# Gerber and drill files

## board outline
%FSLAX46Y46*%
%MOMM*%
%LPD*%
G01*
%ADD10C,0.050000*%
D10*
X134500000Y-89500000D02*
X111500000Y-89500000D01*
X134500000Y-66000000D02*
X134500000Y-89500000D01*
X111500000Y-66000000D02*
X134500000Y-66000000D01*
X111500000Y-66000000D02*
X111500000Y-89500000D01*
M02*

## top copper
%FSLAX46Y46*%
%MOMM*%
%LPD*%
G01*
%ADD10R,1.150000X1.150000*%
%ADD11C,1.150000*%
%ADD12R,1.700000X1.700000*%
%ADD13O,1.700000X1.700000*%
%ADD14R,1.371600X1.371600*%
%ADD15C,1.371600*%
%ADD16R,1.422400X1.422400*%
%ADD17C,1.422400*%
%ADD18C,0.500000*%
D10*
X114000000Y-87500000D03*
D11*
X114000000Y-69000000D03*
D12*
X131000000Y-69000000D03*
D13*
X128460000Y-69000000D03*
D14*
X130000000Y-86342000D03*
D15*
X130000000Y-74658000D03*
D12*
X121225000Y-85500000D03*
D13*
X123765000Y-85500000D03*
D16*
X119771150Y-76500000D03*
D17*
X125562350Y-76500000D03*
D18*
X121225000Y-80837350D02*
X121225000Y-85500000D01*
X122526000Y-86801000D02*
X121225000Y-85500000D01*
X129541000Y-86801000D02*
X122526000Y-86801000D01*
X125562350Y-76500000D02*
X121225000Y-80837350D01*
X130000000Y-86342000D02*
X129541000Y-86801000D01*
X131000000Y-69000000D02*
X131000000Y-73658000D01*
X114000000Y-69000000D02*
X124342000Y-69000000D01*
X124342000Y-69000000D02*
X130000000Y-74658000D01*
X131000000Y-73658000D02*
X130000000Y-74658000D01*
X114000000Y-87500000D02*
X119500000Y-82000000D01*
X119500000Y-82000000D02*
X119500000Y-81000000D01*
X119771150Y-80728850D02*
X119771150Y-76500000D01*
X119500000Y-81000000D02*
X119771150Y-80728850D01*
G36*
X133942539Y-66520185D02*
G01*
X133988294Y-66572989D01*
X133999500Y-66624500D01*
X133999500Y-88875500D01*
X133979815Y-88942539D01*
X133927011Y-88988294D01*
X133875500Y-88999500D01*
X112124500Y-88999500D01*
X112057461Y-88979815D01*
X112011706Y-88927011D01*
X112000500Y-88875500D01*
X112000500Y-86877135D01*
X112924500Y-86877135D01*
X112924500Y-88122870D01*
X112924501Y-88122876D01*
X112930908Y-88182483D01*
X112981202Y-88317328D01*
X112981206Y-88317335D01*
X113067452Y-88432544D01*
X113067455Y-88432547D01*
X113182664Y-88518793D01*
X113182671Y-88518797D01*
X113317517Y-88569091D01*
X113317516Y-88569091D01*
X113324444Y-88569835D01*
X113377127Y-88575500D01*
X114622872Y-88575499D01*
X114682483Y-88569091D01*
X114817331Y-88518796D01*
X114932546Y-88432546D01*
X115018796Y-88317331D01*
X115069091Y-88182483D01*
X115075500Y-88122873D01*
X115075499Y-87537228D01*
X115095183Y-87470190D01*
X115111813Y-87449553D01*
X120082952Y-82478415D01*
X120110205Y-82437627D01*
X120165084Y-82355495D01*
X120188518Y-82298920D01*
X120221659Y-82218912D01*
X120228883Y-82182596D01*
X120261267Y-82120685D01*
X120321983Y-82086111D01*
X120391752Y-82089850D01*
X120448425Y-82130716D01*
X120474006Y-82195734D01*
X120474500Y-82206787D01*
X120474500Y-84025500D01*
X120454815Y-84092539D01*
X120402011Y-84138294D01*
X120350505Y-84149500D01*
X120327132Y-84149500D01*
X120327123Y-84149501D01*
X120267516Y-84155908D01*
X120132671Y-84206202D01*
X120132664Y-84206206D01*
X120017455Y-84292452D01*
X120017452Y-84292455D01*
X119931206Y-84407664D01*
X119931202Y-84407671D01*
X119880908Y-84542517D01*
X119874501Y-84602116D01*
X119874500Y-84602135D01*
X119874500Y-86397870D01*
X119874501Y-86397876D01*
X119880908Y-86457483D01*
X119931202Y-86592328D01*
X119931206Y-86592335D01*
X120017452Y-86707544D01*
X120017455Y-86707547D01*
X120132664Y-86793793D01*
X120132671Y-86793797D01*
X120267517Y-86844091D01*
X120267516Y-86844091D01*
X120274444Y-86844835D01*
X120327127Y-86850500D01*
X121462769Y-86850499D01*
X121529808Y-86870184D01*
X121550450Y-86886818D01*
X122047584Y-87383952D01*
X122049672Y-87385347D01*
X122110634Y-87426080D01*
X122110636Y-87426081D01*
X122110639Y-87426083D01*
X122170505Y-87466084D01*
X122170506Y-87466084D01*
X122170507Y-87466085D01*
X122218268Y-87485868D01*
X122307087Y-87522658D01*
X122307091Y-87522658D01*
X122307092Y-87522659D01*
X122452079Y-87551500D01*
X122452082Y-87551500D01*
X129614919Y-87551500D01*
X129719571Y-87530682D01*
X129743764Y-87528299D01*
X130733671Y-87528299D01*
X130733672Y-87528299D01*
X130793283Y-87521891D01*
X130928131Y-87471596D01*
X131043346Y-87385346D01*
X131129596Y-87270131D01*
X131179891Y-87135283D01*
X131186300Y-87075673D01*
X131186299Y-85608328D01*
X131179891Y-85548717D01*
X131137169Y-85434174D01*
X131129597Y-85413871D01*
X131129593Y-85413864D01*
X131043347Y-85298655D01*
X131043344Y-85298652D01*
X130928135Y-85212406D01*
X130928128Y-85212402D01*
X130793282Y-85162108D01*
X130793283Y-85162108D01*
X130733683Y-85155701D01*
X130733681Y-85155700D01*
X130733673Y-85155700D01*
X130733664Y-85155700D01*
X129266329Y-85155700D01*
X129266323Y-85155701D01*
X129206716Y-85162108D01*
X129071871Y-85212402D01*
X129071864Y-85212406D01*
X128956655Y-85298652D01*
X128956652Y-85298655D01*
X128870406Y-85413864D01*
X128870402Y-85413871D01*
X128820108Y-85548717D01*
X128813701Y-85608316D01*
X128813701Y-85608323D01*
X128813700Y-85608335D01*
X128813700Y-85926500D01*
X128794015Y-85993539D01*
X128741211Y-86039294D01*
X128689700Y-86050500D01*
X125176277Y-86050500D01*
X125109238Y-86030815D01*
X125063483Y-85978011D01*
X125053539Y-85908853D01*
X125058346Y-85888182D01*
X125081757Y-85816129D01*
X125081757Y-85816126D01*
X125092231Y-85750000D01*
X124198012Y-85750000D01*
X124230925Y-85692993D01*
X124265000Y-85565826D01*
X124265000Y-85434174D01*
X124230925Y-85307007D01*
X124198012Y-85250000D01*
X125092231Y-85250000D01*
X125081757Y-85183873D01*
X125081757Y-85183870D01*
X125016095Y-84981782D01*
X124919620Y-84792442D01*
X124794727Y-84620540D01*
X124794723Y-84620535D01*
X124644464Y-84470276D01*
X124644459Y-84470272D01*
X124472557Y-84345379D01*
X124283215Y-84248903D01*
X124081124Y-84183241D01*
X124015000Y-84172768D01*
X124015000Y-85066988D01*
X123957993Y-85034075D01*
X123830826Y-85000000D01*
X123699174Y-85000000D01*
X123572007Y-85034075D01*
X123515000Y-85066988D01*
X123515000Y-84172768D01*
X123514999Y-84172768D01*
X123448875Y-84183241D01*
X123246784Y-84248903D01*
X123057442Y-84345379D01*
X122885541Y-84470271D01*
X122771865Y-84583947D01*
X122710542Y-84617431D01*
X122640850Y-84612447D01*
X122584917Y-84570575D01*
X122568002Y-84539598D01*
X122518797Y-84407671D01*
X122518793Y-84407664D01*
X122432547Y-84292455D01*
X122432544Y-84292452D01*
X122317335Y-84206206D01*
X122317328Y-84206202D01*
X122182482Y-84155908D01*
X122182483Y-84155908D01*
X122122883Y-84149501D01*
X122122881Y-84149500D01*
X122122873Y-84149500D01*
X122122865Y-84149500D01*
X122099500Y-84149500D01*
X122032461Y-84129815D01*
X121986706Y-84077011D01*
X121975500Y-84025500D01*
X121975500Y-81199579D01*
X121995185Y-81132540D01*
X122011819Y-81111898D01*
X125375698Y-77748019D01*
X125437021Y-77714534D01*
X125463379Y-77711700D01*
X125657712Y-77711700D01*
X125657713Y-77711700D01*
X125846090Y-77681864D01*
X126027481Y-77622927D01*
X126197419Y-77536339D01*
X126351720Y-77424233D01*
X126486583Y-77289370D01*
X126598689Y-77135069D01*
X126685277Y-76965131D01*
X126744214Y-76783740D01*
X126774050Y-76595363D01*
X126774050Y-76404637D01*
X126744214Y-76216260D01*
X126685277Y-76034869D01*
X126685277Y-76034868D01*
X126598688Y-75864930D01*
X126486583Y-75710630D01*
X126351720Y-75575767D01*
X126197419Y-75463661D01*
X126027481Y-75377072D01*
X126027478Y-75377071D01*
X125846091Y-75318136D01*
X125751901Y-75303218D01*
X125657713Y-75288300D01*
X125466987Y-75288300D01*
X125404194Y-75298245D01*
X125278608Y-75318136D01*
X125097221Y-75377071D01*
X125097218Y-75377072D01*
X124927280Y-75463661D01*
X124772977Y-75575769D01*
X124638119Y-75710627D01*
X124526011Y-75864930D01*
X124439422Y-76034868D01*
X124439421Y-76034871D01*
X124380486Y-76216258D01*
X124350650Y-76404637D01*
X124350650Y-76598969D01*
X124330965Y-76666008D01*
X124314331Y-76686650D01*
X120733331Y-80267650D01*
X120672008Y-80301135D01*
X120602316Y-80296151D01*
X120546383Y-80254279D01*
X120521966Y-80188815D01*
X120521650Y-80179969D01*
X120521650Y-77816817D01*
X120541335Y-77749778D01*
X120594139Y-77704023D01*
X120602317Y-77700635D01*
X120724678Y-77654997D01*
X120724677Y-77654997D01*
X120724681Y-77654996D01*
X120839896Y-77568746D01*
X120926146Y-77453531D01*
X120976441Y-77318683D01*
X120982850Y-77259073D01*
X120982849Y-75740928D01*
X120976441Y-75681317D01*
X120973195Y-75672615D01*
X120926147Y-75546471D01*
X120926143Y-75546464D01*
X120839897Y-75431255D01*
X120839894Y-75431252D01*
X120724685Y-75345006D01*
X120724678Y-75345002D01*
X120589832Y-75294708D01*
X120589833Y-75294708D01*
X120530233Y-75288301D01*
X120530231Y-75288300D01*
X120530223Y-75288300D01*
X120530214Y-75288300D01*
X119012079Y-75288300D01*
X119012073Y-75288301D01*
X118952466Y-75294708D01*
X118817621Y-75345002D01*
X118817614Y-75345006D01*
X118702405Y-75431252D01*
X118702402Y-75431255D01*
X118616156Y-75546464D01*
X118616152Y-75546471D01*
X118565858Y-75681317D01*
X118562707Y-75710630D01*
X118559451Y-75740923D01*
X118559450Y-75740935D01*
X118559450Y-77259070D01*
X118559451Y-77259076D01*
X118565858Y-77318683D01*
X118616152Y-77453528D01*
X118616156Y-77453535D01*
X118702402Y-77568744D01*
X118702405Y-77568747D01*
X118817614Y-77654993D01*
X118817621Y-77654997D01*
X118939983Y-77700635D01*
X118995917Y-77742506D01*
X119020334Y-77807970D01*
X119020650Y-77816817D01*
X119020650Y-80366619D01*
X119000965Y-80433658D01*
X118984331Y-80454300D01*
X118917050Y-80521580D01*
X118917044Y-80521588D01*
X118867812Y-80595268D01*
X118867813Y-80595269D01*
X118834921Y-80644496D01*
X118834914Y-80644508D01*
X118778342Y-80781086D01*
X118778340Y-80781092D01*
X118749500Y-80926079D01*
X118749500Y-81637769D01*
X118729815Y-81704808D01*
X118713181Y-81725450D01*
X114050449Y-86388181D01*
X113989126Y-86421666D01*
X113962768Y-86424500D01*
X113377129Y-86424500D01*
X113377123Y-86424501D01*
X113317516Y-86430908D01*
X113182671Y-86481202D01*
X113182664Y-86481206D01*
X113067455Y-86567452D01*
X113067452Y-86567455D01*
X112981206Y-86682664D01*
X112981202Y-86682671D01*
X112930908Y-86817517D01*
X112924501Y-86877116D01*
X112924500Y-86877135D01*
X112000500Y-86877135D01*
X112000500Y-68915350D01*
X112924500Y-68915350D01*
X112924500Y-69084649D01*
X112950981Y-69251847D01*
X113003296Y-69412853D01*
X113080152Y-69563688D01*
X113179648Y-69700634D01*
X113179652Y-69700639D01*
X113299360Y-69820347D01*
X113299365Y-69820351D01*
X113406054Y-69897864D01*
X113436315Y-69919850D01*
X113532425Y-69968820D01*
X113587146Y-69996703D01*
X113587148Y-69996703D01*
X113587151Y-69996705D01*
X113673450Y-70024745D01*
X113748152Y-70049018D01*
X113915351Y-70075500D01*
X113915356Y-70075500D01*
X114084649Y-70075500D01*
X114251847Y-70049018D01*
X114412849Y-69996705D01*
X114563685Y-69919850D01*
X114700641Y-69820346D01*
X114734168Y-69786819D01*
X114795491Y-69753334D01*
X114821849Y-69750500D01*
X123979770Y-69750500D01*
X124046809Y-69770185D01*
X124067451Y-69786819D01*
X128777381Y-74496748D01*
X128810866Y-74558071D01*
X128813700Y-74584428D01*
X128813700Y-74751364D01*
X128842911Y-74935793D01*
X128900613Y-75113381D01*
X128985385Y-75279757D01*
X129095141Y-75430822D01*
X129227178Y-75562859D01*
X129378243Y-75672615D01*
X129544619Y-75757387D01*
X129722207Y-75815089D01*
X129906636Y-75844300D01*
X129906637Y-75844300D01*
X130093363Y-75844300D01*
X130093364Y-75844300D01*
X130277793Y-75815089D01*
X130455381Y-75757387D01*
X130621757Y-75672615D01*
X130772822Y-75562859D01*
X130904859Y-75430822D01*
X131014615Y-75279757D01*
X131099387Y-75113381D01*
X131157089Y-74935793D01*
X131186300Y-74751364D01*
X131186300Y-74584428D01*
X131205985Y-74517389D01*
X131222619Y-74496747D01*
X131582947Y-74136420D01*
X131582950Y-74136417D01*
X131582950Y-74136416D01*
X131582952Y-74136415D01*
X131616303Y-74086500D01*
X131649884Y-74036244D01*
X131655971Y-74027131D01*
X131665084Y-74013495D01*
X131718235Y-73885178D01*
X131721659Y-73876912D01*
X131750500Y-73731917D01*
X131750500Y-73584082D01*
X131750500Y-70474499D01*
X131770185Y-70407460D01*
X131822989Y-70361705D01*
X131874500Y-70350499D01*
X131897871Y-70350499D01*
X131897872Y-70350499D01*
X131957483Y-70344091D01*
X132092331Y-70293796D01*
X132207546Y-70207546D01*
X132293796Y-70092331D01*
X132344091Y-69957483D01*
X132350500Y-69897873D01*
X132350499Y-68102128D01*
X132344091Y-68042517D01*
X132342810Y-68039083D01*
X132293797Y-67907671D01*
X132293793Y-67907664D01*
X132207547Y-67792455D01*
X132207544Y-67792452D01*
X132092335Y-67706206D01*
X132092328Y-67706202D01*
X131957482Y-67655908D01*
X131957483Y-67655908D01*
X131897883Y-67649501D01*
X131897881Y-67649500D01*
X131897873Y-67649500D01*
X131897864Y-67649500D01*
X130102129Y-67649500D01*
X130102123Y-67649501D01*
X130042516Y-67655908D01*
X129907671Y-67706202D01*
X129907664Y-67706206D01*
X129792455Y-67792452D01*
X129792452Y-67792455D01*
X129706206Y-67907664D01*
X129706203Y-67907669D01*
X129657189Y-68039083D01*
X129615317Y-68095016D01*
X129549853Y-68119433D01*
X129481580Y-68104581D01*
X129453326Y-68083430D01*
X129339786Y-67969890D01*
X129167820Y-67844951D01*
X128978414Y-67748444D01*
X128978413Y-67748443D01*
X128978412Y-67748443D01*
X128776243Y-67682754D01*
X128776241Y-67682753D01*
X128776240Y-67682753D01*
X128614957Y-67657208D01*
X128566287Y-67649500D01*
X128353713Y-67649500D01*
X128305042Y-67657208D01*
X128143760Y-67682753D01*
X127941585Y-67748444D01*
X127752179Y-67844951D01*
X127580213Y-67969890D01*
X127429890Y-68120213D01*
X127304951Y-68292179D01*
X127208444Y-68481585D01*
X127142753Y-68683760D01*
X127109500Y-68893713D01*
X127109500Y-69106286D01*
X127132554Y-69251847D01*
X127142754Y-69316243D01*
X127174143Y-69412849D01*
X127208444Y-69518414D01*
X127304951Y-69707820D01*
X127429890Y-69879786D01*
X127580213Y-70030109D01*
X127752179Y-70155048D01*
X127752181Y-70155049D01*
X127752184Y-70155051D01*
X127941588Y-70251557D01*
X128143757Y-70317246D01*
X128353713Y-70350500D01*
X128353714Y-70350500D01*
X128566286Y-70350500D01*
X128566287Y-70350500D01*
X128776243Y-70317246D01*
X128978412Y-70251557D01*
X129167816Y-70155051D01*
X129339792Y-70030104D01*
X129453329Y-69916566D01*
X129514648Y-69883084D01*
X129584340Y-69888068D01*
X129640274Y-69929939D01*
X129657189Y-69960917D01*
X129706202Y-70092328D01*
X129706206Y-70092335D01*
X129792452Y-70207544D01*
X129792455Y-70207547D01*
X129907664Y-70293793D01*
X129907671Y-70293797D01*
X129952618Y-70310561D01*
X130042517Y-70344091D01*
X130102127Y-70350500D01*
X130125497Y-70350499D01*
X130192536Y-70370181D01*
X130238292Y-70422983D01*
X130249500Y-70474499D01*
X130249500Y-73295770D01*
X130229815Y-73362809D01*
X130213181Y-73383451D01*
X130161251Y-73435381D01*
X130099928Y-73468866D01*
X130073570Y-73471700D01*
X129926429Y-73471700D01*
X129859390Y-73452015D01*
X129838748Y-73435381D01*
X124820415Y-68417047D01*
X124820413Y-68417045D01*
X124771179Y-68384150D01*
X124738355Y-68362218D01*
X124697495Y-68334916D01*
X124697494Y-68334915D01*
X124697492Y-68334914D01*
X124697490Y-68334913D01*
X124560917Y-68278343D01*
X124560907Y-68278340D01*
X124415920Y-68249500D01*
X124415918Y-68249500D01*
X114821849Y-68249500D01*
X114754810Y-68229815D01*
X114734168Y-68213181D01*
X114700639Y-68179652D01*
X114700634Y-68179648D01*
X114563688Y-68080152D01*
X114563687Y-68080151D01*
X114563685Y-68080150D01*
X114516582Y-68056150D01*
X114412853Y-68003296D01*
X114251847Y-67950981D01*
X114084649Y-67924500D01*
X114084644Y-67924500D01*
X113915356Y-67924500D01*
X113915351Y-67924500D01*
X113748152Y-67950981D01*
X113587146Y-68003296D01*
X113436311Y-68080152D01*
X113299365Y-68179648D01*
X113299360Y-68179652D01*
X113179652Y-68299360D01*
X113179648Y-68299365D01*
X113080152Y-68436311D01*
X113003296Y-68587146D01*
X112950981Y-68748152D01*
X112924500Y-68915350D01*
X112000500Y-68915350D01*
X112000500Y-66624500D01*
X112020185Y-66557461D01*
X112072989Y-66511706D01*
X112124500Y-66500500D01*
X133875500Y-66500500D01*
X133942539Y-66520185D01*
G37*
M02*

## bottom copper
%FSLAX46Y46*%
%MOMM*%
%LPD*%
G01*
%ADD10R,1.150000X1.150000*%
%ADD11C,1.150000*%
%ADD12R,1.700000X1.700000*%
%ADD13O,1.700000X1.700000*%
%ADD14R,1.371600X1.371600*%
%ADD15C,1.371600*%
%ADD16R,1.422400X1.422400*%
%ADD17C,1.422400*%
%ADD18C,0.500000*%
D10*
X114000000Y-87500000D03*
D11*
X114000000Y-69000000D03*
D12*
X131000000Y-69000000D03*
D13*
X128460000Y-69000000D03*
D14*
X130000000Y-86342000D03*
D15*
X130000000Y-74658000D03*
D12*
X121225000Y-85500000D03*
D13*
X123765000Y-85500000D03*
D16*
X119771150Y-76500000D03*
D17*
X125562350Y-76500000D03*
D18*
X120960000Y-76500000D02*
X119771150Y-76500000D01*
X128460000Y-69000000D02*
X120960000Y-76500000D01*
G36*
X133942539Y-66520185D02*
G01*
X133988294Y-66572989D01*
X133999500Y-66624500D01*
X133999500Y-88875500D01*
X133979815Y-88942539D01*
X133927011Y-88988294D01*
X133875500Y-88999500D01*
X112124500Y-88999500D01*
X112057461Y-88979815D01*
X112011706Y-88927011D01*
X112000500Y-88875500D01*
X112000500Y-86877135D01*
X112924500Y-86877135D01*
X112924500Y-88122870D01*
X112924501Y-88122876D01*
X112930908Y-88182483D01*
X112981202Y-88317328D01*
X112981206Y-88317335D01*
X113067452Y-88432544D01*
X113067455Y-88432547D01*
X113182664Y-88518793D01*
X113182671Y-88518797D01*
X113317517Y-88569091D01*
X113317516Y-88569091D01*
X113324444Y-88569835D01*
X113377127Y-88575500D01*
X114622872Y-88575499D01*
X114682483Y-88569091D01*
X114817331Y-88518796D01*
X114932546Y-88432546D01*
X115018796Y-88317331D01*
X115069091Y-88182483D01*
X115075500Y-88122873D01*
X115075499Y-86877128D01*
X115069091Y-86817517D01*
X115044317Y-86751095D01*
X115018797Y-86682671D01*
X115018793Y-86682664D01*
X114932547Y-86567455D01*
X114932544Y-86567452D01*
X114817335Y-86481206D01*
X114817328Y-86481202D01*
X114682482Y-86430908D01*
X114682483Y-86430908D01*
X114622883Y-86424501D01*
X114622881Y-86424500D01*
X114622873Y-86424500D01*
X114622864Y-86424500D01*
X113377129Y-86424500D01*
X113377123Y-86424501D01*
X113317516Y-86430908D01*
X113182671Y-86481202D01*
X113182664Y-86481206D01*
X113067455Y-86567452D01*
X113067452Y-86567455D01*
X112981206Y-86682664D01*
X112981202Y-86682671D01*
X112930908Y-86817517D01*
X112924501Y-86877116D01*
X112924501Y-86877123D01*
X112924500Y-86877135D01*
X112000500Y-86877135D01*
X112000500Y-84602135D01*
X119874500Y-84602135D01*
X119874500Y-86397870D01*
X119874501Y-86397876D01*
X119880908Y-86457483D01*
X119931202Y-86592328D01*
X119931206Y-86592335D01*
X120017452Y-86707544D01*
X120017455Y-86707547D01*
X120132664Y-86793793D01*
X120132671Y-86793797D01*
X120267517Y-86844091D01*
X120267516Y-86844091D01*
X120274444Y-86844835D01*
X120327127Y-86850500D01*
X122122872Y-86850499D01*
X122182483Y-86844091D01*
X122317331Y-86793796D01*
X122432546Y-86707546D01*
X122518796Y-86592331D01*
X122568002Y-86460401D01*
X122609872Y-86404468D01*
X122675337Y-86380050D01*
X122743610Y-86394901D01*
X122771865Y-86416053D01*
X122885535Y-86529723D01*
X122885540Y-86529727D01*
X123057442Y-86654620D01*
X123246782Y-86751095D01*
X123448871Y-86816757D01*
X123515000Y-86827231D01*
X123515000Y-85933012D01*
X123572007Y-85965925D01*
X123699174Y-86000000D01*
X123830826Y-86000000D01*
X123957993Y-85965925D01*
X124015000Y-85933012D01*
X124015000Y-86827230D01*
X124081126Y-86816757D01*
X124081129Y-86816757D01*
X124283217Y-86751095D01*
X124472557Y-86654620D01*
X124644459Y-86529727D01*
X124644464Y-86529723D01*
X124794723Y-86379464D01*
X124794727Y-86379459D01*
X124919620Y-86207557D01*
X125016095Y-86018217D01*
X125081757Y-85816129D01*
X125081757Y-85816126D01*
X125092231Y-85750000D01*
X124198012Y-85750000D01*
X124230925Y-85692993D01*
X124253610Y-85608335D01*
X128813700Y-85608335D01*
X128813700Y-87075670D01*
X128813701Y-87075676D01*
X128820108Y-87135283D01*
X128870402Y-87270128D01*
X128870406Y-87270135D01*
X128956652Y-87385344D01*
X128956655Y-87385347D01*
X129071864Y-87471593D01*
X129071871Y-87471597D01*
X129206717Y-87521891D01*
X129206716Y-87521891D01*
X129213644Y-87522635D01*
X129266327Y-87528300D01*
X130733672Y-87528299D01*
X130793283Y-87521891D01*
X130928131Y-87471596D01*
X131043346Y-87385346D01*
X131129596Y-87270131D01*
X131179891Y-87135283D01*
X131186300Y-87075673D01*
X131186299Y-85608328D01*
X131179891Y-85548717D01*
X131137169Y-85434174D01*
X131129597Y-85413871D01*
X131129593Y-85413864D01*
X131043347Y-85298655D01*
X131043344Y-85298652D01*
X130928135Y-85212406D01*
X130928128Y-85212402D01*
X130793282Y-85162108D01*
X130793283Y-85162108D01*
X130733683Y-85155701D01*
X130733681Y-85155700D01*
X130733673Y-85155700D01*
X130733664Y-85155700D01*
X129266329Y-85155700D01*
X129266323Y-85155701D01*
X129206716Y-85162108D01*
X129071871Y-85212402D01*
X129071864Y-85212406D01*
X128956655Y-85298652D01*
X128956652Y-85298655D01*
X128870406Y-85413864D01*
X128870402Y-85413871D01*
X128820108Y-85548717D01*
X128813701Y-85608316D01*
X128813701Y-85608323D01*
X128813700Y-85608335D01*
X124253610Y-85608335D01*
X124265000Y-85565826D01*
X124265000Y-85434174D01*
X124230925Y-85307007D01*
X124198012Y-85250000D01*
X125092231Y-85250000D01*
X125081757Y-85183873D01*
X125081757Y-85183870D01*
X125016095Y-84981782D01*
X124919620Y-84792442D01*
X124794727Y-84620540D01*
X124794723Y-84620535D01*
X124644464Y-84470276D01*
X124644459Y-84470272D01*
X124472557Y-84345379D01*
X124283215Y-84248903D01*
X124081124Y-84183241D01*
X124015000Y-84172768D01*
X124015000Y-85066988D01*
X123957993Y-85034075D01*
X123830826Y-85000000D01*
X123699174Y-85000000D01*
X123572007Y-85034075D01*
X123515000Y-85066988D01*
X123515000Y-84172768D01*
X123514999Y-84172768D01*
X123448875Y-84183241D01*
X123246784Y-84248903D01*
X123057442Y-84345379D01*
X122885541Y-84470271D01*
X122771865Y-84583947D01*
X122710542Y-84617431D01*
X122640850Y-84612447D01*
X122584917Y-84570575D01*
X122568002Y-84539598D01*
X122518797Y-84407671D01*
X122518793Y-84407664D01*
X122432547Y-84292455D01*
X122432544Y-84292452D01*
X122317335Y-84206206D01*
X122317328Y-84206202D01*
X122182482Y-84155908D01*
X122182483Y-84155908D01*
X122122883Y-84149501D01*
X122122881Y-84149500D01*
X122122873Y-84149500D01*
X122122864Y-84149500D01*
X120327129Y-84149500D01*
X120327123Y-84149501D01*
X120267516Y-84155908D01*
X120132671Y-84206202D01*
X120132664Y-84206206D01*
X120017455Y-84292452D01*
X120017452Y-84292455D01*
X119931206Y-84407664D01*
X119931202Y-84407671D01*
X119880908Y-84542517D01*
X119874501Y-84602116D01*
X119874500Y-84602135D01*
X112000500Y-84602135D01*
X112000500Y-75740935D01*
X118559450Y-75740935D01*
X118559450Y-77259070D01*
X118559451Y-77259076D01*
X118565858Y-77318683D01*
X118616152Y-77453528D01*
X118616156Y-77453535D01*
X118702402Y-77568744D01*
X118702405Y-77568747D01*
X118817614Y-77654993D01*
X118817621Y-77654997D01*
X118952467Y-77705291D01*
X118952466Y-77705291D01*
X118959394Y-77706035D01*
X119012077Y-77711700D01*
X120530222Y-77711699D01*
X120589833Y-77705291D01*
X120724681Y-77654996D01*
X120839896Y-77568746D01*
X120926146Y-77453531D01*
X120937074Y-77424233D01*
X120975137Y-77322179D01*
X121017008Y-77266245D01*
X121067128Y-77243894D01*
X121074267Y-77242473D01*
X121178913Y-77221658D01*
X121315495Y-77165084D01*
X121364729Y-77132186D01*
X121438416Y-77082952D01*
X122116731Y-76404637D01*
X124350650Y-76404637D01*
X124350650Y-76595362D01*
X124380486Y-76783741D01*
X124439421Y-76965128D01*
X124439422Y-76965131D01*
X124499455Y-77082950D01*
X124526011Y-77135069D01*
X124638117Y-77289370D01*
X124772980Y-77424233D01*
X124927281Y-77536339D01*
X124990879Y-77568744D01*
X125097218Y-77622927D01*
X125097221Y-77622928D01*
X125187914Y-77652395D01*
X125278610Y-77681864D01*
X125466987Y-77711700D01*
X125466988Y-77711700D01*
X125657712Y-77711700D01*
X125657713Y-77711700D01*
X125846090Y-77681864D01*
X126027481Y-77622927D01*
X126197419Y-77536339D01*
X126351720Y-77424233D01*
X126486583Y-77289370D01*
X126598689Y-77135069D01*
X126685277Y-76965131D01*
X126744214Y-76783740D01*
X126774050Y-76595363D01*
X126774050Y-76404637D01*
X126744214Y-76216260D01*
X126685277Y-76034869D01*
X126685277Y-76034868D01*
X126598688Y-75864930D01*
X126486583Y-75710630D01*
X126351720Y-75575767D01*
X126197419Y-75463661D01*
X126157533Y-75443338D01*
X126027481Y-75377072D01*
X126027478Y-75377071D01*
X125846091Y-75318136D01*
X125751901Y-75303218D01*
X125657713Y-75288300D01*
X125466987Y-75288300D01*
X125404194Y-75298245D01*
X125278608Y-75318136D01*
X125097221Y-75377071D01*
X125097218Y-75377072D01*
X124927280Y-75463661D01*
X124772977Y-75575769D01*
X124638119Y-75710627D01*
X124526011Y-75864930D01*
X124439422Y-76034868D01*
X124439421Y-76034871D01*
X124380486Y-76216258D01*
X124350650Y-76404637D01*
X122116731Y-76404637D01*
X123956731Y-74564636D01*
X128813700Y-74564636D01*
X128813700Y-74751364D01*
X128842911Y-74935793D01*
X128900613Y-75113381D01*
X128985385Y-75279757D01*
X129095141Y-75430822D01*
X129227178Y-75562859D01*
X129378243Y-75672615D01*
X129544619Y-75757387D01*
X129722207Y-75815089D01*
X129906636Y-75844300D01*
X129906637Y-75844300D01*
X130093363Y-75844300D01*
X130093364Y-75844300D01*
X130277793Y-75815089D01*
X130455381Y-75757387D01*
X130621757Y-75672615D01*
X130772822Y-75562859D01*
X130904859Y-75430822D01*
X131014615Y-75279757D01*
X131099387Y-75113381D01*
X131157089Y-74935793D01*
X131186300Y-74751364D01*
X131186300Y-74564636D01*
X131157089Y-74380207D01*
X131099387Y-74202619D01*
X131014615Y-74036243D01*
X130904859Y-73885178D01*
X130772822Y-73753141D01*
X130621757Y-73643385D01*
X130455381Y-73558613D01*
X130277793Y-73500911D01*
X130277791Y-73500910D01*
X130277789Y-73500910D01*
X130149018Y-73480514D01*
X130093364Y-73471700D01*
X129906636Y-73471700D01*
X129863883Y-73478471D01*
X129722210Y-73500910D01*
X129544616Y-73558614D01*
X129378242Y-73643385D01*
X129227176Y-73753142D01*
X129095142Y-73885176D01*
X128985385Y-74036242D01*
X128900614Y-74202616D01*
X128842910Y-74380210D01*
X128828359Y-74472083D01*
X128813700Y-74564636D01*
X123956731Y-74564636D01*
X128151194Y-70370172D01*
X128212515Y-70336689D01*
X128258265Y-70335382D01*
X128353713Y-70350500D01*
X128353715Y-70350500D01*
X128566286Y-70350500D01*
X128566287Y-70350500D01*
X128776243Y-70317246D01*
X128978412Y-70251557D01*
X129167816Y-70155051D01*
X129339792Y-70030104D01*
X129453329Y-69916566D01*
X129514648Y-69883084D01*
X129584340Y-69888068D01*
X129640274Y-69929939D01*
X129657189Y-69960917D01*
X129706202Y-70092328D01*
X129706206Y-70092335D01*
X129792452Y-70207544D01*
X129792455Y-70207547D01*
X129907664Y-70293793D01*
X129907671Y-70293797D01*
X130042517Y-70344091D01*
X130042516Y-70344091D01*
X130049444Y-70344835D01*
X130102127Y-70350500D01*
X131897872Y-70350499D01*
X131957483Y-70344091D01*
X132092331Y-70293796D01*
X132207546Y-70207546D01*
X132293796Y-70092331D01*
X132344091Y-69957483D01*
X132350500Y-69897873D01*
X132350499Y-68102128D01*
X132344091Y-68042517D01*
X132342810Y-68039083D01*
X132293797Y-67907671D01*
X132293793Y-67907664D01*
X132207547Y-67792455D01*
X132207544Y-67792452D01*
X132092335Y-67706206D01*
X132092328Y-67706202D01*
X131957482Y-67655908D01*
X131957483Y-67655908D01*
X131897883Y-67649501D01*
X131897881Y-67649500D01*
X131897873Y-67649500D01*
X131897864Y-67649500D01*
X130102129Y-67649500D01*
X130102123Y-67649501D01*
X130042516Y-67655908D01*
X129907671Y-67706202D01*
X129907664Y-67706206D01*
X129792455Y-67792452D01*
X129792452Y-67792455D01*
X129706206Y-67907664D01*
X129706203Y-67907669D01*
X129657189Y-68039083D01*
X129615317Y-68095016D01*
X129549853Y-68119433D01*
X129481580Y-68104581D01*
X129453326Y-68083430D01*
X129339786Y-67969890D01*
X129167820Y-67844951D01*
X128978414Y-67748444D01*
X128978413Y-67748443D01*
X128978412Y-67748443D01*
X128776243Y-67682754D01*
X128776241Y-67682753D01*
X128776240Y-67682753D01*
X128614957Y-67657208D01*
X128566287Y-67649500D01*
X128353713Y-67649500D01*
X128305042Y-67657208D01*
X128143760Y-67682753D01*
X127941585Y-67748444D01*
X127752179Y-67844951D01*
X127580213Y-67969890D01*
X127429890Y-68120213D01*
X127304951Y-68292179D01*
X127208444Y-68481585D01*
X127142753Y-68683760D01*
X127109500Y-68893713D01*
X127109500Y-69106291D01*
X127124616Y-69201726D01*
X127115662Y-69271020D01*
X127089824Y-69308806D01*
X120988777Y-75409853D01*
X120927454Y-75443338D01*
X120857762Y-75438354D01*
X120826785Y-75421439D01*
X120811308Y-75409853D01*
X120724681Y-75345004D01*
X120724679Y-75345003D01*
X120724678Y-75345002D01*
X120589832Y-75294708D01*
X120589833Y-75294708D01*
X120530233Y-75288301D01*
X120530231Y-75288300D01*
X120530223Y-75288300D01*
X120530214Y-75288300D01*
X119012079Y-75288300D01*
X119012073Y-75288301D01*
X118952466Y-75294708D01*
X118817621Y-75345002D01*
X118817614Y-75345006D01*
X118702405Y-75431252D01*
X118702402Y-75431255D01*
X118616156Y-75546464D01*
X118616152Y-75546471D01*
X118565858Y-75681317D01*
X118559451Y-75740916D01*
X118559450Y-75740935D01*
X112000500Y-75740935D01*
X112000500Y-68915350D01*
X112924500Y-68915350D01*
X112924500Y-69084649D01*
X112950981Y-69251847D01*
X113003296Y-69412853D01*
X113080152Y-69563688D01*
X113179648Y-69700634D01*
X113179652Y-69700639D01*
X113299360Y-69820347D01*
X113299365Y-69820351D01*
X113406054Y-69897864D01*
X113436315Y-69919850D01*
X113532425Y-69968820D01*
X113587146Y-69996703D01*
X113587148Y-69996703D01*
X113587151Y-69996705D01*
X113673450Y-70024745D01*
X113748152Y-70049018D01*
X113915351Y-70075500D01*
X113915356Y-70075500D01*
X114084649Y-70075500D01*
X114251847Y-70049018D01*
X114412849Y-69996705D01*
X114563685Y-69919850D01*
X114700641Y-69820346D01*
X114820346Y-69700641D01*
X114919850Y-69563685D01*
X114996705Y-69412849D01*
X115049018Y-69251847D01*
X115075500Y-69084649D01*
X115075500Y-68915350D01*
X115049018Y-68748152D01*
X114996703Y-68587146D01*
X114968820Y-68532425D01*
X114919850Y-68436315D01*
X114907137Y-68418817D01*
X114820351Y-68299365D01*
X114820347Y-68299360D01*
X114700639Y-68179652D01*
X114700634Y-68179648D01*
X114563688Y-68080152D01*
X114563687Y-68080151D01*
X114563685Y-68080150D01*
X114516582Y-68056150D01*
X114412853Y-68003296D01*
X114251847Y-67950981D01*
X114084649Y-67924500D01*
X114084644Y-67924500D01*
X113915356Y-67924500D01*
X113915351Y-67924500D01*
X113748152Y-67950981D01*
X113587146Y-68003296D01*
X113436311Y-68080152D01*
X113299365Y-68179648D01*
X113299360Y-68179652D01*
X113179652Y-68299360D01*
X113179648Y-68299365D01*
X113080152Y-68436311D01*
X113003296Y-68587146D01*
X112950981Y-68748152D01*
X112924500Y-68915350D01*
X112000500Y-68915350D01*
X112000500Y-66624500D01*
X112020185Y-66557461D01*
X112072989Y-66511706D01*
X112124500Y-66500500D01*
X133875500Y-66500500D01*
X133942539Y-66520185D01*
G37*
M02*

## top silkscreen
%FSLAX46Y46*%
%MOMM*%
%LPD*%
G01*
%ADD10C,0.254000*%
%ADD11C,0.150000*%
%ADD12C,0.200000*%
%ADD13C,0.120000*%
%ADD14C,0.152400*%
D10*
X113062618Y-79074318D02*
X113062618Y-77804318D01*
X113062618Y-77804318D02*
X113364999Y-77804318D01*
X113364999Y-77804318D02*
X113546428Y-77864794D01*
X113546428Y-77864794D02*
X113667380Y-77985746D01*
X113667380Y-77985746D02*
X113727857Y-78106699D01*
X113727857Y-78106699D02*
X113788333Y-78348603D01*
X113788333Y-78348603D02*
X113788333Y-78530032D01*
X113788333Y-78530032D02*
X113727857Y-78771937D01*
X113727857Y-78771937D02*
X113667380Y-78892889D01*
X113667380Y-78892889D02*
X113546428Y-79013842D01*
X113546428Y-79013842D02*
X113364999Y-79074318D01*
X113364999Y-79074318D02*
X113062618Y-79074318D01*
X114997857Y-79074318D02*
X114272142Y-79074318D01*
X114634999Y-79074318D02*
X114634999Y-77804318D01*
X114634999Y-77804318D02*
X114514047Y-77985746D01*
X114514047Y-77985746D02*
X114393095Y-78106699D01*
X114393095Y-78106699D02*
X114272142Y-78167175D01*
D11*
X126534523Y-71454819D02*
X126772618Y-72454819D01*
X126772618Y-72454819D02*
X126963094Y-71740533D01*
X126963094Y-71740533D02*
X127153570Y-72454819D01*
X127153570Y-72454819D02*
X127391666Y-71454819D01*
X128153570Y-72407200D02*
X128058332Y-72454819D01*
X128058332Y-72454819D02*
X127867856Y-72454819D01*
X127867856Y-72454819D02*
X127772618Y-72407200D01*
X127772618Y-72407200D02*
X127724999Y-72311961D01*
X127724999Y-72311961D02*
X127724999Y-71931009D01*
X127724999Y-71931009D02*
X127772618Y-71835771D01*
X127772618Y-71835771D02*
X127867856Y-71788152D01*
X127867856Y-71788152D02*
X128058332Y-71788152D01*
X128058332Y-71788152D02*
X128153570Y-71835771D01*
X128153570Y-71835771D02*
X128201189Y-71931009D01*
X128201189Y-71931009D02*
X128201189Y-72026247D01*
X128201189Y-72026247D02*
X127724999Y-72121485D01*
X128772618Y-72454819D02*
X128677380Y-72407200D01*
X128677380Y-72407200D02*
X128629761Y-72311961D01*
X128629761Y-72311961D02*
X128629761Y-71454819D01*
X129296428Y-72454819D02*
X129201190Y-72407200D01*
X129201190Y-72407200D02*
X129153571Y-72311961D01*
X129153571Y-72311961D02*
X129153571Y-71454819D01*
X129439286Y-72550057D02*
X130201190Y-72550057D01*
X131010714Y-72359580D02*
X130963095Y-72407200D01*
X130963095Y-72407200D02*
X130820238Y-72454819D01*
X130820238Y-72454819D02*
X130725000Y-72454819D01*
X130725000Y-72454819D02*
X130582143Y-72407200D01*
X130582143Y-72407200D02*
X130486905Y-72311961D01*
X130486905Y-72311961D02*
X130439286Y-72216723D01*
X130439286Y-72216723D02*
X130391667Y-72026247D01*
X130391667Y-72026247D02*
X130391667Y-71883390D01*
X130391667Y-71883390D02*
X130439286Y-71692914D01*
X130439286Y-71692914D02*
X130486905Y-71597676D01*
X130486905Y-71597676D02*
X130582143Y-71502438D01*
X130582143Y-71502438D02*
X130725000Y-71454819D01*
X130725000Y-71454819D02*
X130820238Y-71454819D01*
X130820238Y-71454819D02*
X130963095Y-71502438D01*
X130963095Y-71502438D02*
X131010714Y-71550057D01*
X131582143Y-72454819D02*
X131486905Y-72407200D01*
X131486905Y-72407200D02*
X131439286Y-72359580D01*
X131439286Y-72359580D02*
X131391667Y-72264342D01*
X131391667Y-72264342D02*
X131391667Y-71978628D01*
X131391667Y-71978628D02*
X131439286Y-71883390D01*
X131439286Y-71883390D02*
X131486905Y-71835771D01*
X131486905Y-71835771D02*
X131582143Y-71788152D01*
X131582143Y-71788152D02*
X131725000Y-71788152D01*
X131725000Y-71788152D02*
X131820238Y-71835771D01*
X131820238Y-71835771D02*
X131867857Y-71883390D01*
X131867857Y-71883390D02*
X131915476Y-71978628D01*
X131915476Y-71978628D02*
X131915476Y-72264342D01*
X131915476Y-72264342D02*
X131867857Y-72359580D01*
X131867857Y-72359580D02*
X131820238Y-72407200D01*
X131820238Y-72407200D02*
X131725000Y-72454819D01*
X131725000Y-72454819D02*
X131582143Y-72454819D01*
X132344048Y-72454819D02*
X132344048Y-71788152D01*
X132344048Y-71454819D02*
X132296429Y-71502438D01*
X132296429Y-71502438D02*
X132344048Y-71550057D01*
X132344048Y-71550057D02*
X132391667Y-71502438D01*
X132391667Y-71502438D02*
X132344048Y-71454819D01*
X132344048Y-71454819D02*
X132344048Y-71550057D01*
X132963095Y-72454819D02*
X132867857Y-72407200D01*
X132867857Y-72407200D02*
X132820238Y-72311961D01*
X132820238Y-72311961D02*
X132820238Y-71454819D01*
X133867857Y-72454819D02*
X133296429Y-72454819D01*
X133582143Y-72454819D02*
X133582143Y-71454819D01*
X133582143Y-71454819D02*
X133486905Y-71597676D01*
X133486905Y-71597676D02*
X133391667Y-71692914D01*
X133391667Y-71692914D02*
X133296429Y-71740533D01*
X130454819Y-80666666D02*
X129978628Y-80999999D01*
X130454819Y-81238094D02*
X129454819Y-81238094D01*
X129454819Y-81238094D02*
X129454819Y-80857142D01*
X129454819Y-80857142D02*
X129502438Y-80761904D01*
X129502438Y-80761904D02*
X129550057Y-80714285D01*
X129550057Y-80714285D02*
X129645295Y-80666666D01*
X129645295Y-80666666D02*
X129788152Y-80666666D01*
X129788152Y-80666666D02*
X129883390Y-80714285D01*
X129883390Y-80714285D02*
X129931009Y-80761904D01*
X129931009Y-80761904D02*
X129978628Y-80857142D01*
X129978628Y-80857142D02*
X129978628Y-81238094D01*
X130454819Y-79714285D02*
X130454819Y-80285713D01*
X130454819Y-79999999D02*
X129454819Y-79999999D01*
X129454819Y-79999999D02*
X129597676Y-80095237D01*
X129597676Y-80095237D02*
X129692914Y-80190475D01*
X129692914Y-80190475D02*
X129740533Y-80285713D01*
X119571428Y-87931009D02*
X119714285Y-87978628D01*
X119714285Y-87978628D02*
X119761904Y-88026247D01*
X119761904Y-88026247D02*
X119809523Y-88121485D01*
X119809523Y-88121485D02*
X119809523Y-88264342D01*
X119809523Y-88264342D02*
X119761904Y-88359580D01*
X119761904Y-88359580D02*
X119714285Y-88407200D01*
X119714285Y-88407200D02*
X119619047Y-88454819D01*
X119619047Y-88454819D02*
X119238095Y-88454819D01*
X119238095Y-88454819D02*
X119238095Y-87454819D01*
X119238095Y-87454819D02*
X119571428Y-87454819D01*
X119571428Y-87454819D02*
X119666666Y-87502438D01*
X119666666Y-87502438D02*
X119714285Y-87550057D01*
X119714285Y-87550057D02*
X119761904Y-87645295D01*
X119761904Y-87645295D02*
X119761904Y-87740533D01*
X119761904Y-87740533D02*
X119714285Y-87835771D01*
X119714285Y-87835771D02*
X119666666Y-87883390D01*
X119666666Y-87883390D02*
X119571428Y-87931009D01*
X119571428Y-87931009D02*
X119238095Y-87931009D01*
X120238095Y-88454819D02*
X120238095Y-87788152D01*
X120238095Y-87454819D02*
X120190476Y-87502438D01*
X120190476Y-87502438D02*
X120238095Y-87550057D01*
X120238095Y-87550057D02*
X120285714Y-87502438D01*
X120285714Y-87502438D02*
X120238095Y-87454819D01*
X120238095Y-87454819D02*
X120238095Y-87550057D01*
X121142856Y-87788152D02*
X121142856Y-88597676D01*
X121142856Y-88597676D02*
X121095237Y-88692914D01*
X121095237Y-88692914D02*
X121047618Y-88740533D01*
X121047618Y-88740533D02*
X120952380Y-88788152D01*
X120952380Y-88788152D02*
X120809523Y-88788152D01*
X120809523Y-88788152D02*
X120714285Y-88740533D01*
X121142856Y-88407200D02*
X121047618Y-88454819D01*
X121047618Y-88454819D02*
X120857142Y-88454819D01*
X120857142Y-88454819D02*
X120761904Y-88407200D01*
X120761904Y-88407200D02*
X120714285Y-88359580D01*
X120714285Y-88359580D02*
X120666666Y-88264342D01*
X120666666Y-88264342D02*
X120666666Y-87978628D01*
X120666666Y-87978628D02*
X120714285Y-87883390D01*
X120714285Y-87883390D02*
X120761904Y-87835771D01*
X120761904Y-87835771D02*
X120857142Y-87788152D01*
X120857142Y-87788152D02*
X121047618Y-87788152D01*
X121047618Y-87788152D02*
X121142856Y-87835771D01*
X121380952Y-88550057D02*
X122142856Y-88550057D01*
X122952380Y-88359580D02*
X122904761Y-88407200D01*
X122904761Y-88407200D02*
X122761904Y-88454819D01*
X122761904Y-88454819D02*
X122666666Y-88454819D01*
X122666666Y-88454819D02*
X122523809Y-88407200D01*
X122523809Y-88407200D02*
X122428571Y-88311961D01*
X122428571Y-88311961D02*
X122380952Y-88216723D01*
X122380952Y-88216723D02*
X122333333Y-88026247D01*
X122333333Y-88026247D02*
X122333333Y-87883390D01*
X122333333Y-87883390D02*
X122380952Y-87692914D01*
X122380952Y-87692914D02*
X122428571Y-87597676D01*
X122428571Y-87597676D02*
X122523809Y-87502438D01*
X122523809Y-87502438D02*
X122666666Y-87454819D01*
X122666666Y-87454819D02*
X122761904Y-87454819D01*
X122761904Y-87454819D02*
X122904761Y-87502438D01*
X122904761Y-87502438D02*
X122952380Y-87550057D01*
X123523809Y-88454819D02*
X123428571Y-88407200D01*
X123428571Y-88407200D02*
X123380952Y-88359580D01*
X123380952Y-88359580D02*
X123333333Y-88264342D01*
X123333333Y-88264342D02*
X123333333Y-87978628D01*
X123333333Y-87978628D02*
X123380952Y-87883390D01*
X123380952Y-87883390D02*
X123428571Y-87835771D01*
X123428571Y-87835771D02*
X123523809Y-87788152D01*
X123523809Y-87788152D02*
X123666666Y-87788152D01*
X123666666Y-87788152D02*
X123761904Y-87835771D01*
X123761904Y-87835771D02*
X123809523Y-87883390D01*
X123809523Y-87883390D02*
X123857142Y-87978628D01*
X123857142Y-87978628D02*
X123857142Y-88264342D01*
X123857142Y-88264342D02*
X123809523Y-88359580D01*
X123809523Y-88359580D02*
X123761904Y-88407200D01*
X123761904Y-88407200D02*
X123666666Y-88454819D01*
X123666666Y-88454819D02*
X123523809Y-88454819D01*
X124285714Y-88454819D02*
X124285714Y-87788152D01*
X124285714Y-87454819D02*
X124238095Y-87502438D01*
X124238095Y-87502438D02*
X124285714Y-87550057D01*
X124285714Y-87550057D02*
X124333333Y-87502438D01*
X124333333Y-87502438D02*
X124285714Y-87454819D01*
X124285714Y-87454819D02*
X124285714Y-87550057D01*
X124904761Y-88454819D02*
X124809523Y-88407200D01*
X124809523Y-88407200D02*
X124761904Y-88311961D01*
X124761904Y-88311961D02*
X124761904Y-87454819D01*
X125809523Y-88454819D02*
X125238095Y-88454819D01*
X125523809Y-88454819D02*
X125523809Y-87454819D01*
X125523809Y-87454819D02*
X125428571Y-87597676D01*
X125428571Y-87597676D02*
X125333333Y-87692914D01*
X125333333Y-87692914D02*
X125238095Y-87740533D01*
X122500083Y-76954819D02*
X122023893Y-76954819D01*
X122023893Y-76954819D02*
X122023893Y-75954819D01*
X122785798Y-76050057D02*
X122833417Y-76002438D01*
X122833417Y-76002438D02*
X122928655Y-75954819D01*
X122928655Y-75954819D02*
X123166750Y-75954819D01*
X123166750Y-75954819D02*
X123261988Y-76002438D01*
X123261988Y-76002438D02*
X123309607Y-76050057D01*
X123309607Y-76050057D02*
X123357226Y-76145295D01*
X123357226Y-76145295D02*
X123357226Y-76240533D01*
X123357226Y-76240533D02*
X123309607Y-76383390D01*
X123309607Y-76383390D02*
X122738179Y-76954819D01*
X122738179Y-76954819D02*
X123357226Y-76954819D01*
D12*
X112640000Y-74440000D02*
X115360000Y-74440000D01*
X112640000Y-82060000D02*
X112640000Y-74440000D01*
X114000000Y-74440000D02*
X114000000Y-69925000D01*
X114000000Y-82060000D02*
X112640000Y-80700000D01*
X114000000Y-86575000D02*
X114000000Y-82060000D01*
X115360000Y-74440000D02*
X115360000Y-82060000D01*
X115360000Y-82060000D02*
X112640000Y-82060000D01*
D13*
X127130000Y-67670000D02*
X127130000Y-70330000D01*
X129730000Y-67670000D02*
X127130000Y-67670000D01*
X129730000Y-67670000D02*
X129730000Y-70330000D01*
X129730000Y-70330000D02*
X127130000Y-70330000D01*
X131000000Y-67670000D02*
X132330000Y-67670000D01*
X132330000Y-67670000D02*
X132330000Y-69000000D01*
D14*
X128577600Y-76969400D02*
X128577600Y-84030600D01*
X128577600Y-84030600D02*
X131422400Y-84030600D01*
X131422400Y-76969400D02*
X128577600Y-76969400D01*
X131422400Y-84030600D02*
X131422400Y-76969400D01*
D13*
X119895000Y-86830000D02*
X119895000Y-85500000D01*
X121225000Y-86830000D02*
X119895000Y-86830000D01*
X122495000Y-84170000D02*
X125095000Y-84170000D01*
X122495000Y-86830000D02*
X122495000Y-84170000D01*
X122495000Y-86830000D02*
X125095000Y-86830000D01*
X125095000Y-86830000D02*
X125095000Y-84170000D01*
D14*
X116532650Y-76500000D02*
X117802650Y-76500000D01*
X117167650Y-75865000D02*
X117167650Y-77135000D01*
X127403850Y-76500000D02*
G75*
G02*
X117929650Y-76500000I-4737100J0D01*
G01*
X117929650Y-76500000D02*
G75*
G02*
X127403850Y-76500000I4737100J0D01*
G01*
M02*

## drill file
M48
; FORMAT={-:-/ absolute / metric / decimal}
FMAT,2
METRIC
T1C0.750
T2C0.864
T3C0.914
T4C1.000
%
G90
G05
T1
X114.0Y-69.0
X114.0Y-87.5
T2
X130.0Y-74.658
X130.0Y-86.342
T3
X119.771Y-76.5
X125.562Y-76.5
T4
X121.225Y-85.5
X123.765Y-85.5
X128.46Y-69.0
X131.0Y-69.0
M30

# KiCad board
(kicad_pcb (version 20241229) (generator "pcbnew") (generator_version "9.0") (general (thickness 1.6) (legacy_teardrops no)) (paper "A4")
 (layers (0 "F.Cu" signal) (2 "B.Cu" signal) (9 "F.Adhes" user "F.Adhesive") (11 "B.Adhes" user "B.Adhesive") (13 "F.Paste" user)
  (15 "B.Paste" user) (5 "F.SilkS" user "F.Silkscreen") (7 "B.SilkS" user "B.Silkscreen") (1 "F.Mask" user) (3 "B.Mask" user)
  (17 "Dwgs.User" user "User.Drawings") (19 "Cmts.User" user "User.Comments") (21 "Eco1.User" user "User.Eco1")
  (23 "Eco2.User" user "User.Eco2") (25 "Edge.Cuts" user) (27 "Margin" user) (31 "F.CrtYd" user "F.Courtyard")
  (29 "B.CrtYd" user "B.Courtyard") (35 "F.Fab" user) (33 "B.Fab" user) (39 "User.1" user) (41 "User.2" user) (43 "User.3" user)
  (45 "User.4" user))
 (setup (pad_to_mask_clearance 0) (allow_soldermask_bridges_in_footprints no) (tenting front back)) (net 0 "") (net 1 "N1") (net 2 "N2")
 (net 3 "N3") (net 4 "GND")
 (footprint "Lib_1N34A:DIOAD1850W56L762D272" (layer "F.Cu") (at 114 87.5 90)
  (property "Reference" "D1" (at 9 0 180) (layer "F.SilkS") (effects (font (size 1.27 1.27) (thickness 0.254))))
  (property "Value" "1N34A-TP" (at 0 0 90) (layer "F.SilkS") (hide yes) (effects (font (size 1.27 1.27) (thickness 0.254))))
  (fp_line (start 13.06 -1.36) (end 13.06 1.36) (stroke (width 0.2) (type solid)) (layer "F.SilkS"))
  (fp_line (start 5.44 -1.36) (end 13.06 -1.36) (stroke (width 0.2) (type solid)) (layer "F.SilkS"))
  (fp_line (start 13.06 0) (end 17.575 0) (stroke (width 0.2) (type solid)) (layer "F.SilkS"))
  (fp_line (start 5.44 0) (end 6.8 -1.36) (stroke (width 0.2) (type solid)) (layer "F.SilkS"))
  (fp_line (start 0.925 0) (end 5.44 0) (stroke (width 0.2) (type solid)) (layer "F.SilkS"))
  (fp_line (start 13.06 1.36) (end 5.44 1.36) (stroke (width 0.2) (type solid)) (layer "F.SilkS"))
  (fp_line (start 5.44 1.36) (end 5.44 -1.36) (stroke (width 0.2) (type solid)) (layer "F.SilkS"))
  (pad "1" thru_hole rect (at 0 0 90) (size 1.15 1.15) (drill 0.75) (layers "*.Cu" "*.Mask") (remove_unused_layers no) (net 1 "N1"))
  (pad "2" thru_hole circle (at 18.5 0 90) (size 1.15 1.15) (drill 0.75) (layers "*.Cu" "*.Mask") (remove_unused_layers no) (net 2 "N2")))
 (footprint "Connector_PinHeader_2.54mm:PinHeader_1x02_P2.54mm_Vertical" (layer "F.Cu") (at 131 69 -90)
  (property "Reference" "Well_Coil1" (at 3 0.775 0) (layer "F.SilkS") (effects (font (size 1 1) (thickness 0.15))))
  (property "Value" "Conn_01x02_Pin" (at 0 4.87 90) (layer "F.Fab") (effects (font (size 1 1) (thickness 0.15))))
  (fp_line (start -1.33 3.87) (end 1.33 3.87) (stroke (width 0.12) (type solid)) (layer "F.SilkS"))
  (fp_line (start -1.33 1.27) (end -1.33 3.87) (stroke (width 0.12) (type solid)) (layer "F.SilkS"))
  (fp_line (start -1.33 1.27) (end 1.33 1.27) (stroke (width 0.12) (type solid)) (layer "F.SilkS"))
  (fp_line (start 1.33 1.27) (end 1.33 3.87) (stroke (width 0.12) (type solid)) (layer "F.SilkS"))
  (fp_line (start -1.33 0) (end -1.33 -1.33) (stroke (width 0.12) (type solid)) (layer "F.SilkS"))
  (fp_line (start -1.33 -1.33) (end 0 -1.33) (stroke (width 0.12) (type solid)) (layer "F.SilkS"))
  (pad "1" thru_hole rect (at 0 0 270) (size 1.7 1.7) (drill 1) (layers "*.Cu" "*.Mask") (remove_unused_layers no) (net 2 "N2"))
  (pad "2" thru_hole oval (at 0 2.54 270) (size 1.7 1.7) (drill 1) (layers "*.Cu" "*.Mask") (remove_unused_layers no) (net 1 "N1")))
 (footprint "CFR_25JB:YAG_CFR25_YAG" (layer "F.Cu") (at 130 86.342 90)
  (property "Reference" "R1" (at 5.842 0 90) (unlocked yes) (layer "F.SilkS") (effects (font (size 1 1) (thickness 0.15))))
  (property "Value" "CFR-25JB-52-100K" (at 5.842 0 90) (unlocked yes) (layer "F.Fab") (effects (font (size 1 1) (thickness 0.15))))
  (fp_line (start 9.3726 -1.4224) (end 2.3114 -1.4224) (stroke (width 0.1524) (type solid)) (layer "F.SilkS"))
  (fp_line (start 2.3114 -1.4224) (end 2.3114 1.4224) (stroke (width 0.1524) (type solid)) (layer "F.SilkS"))
  (fp_line (start 9.3726 1.4224) (end 9.3726 -1.4224) (stroke (width 0.1524) (type solid)) (layer "F.SilkS"))
  (fp_line (start 2.3114 1.4224) (end 9.3726 1.4224) (stroke (width 0.1524) (type solid)) (layer "F.SilkS"))
  (pad "1" thru_hole rect (at 0 0 90) (size 1.3716 1.3716) (drill 0.8636) (layers "*.Cu" "*.Mask") (remove_unused_layers no) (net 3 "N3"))
  (pad "2" thru_hole circle (at 11.684 0 90) (size 1.3716 1.3716) (drill 0.8636) (layers "*.Cu" "*.Mask") (remove_unused_layers no)
   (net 2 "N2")))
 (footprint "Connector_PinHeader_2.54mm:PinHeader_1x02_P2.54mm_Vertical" (layer "F.Cu") (at 121.225 85.5 90)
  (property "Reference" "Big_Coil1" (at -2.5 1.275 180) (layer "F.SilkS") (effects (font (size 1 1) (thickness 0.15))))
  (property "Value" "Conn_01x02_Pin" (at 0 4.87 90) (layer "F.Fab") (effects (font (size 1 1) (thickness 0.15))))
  (fp_line (start -1.33 -1.33) (end 0 -1.33) (stroke (width 0.12) (type solid)) (layer "F.SilkS"))
  (fp_line (start -1.33 0) (end -1.33 -1.33) (stroke (width 0.12) (type solid)) (layer "F.SilkS"))
  (fp_line (start 1.33 1.27) (end 1.33 3.87) (stroke (width 0.12) (type solid)) (layer "F.SilkS"))
  (fp_line (start -1.33 1.27) (end 1.33 1.27) (stroke (width 0.12) (type solid)) (layer "F.SilkS"))
  (fp_line (start -1.33 1.27) (end -1.33 3.87) (stroke (width 0.12) (type solid)) (layer "F.SilkS"))
  (fp_line (start -1.33 3.87) (end 1.33 3.87) (stroke (width 0.12) (type solid)) (layer "F.SilkS"))
  (pad "1" thru_hole rect (at 0 0 90) (size 1.7 1.7) (drill 1) (layers "*.Cu" "*.Mask") (remove_unused_layers no) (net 3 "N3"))
  (pad "2" thru_hole oval (at 0 2.54 90) (size 1.7 1.7) (drill 1) (layers "*.Cu" "*.Mask") (remove_unused_layers no) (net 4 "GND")))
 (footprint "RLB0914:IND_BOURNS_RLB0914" (layer "F.Cu") (at 119.77115 76.5)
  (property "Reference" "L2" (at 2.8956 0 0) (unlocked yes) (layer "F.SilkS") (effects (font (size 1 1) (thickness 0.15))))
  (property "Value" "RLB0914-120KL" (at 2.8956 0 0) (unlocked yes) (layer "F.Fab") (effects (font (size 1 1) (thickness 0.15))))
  (fp_line (start -3.2385 0) (end -1.9685 0) (stroke (width 0.1524) (type solid)) (layer "F.SilkS"))
  (fp_line (start -2.6035 -0.635) (end -2.6035 0.635) (stroke (width 0.1524) (type solid)) (layer "F.SilkS"))
  (fp_circle (center 2.8956 0) (end 7.6327 0) (stroke (width 0.1524) (type solid)) (fill no) (layer "F.SilkS"))
  (pad "1" thru_hole rect (at 0 0) (size 1.4224 1.4224) (drill 0.9144) (layers "*.Cu" "*.Mask") (remove_unused_layers no) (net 1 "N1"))
  (pad "2" thru_hole circle (at 5.7912 0) (size 1.4224 1.4224) (drill 0.9144) (layers "*.Cu" "*.Mask") (remove_unused_layers no)
   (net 3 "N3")))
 (gr_line (start 134.5 89.5) (end 111.5 89.5) (stroke (width 0.05) (type default)) (layer "Edge.Cuts"))
 (gr_line (start 134.5 66) (end 134.5 89.5) (stroke (width 0.05) (type default)) (layer "Edge.Cuts"))
 (gr_line (start 111.5 66) (end 134.5 66) (stroke (width 0.05) (type default)) (layer "Edge.Cuts"))
 (gr_line (start 111.5 66) (end 111.5 89.5) (stroke (width 0.05) (type default)) (layer "Edge.Cuts"))
 (segment (start 121.225 80.83735) (end 121.225 85.5) (width 0.5) (layer "F.Cu") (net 3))
 (segment (start 122.526 86.801) (end 121.225 85.5) (width 0.5) (layer "F.Cu") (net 3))
 (segment (start 129.541 86.801) (end 122.526 86.801) (width 0.5) (layer "F.Cu") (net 3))
 (segment (start 125.56235 76.5) (end 121.225 80.83735) (width 0.5) (layer "F.Cu") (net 3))
 (segment (start 130 86.342) (end 129.541 86.801) (width 0.5) (layer "F.Cu") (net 3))
 (segment (start 131 69) (end 131 73.658) (width 0.5) (layer "F.Cu") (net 2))
 (segment (start 114 69) (end 124.342 69) (width 0.5) (layer "F.Cu") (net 2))
 (segment (start 124.342 69) (end 130 74.658) (width 0.5) (layer "F.Cu") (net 2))
 (segment (start 131 73.658) (end 130 74.658) (width 0.5) (layer "F.Cu") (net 2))
 (segment (start 114 87.5) (end 119.5 82) (width 0.5) (layer "F.Cu") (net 1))
 (segment (start 119.5 82) (end 119.5 81) (width 0.5) (layer "F.Cu") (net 1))
 (segment (start 119.77115 80.72885) (end 119.77115 76.5) (width 0.5) (layer "F.Cu") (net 1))
 (segment (start 119.5 81) (end 119.77115 80.72885) (width 0.5) (layer "F.Cu") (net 1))
 (segment (start 120.96 76.5) (end 119.77115 76.5) (width 0.5) (layer "B.Cu") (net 1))
 (segment (start 128.46 69) (end 120.96 76.5) (width 0.5) (layer "B.Cu") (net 1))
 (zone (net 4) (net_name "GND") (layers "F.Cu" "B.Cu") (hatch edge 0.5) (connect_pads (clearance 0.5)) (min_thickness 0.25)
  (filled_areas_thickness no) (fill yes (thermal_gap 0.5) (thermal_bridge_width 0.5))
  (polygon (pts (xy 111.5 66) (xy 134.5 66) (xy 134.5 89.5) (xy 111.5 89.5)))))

